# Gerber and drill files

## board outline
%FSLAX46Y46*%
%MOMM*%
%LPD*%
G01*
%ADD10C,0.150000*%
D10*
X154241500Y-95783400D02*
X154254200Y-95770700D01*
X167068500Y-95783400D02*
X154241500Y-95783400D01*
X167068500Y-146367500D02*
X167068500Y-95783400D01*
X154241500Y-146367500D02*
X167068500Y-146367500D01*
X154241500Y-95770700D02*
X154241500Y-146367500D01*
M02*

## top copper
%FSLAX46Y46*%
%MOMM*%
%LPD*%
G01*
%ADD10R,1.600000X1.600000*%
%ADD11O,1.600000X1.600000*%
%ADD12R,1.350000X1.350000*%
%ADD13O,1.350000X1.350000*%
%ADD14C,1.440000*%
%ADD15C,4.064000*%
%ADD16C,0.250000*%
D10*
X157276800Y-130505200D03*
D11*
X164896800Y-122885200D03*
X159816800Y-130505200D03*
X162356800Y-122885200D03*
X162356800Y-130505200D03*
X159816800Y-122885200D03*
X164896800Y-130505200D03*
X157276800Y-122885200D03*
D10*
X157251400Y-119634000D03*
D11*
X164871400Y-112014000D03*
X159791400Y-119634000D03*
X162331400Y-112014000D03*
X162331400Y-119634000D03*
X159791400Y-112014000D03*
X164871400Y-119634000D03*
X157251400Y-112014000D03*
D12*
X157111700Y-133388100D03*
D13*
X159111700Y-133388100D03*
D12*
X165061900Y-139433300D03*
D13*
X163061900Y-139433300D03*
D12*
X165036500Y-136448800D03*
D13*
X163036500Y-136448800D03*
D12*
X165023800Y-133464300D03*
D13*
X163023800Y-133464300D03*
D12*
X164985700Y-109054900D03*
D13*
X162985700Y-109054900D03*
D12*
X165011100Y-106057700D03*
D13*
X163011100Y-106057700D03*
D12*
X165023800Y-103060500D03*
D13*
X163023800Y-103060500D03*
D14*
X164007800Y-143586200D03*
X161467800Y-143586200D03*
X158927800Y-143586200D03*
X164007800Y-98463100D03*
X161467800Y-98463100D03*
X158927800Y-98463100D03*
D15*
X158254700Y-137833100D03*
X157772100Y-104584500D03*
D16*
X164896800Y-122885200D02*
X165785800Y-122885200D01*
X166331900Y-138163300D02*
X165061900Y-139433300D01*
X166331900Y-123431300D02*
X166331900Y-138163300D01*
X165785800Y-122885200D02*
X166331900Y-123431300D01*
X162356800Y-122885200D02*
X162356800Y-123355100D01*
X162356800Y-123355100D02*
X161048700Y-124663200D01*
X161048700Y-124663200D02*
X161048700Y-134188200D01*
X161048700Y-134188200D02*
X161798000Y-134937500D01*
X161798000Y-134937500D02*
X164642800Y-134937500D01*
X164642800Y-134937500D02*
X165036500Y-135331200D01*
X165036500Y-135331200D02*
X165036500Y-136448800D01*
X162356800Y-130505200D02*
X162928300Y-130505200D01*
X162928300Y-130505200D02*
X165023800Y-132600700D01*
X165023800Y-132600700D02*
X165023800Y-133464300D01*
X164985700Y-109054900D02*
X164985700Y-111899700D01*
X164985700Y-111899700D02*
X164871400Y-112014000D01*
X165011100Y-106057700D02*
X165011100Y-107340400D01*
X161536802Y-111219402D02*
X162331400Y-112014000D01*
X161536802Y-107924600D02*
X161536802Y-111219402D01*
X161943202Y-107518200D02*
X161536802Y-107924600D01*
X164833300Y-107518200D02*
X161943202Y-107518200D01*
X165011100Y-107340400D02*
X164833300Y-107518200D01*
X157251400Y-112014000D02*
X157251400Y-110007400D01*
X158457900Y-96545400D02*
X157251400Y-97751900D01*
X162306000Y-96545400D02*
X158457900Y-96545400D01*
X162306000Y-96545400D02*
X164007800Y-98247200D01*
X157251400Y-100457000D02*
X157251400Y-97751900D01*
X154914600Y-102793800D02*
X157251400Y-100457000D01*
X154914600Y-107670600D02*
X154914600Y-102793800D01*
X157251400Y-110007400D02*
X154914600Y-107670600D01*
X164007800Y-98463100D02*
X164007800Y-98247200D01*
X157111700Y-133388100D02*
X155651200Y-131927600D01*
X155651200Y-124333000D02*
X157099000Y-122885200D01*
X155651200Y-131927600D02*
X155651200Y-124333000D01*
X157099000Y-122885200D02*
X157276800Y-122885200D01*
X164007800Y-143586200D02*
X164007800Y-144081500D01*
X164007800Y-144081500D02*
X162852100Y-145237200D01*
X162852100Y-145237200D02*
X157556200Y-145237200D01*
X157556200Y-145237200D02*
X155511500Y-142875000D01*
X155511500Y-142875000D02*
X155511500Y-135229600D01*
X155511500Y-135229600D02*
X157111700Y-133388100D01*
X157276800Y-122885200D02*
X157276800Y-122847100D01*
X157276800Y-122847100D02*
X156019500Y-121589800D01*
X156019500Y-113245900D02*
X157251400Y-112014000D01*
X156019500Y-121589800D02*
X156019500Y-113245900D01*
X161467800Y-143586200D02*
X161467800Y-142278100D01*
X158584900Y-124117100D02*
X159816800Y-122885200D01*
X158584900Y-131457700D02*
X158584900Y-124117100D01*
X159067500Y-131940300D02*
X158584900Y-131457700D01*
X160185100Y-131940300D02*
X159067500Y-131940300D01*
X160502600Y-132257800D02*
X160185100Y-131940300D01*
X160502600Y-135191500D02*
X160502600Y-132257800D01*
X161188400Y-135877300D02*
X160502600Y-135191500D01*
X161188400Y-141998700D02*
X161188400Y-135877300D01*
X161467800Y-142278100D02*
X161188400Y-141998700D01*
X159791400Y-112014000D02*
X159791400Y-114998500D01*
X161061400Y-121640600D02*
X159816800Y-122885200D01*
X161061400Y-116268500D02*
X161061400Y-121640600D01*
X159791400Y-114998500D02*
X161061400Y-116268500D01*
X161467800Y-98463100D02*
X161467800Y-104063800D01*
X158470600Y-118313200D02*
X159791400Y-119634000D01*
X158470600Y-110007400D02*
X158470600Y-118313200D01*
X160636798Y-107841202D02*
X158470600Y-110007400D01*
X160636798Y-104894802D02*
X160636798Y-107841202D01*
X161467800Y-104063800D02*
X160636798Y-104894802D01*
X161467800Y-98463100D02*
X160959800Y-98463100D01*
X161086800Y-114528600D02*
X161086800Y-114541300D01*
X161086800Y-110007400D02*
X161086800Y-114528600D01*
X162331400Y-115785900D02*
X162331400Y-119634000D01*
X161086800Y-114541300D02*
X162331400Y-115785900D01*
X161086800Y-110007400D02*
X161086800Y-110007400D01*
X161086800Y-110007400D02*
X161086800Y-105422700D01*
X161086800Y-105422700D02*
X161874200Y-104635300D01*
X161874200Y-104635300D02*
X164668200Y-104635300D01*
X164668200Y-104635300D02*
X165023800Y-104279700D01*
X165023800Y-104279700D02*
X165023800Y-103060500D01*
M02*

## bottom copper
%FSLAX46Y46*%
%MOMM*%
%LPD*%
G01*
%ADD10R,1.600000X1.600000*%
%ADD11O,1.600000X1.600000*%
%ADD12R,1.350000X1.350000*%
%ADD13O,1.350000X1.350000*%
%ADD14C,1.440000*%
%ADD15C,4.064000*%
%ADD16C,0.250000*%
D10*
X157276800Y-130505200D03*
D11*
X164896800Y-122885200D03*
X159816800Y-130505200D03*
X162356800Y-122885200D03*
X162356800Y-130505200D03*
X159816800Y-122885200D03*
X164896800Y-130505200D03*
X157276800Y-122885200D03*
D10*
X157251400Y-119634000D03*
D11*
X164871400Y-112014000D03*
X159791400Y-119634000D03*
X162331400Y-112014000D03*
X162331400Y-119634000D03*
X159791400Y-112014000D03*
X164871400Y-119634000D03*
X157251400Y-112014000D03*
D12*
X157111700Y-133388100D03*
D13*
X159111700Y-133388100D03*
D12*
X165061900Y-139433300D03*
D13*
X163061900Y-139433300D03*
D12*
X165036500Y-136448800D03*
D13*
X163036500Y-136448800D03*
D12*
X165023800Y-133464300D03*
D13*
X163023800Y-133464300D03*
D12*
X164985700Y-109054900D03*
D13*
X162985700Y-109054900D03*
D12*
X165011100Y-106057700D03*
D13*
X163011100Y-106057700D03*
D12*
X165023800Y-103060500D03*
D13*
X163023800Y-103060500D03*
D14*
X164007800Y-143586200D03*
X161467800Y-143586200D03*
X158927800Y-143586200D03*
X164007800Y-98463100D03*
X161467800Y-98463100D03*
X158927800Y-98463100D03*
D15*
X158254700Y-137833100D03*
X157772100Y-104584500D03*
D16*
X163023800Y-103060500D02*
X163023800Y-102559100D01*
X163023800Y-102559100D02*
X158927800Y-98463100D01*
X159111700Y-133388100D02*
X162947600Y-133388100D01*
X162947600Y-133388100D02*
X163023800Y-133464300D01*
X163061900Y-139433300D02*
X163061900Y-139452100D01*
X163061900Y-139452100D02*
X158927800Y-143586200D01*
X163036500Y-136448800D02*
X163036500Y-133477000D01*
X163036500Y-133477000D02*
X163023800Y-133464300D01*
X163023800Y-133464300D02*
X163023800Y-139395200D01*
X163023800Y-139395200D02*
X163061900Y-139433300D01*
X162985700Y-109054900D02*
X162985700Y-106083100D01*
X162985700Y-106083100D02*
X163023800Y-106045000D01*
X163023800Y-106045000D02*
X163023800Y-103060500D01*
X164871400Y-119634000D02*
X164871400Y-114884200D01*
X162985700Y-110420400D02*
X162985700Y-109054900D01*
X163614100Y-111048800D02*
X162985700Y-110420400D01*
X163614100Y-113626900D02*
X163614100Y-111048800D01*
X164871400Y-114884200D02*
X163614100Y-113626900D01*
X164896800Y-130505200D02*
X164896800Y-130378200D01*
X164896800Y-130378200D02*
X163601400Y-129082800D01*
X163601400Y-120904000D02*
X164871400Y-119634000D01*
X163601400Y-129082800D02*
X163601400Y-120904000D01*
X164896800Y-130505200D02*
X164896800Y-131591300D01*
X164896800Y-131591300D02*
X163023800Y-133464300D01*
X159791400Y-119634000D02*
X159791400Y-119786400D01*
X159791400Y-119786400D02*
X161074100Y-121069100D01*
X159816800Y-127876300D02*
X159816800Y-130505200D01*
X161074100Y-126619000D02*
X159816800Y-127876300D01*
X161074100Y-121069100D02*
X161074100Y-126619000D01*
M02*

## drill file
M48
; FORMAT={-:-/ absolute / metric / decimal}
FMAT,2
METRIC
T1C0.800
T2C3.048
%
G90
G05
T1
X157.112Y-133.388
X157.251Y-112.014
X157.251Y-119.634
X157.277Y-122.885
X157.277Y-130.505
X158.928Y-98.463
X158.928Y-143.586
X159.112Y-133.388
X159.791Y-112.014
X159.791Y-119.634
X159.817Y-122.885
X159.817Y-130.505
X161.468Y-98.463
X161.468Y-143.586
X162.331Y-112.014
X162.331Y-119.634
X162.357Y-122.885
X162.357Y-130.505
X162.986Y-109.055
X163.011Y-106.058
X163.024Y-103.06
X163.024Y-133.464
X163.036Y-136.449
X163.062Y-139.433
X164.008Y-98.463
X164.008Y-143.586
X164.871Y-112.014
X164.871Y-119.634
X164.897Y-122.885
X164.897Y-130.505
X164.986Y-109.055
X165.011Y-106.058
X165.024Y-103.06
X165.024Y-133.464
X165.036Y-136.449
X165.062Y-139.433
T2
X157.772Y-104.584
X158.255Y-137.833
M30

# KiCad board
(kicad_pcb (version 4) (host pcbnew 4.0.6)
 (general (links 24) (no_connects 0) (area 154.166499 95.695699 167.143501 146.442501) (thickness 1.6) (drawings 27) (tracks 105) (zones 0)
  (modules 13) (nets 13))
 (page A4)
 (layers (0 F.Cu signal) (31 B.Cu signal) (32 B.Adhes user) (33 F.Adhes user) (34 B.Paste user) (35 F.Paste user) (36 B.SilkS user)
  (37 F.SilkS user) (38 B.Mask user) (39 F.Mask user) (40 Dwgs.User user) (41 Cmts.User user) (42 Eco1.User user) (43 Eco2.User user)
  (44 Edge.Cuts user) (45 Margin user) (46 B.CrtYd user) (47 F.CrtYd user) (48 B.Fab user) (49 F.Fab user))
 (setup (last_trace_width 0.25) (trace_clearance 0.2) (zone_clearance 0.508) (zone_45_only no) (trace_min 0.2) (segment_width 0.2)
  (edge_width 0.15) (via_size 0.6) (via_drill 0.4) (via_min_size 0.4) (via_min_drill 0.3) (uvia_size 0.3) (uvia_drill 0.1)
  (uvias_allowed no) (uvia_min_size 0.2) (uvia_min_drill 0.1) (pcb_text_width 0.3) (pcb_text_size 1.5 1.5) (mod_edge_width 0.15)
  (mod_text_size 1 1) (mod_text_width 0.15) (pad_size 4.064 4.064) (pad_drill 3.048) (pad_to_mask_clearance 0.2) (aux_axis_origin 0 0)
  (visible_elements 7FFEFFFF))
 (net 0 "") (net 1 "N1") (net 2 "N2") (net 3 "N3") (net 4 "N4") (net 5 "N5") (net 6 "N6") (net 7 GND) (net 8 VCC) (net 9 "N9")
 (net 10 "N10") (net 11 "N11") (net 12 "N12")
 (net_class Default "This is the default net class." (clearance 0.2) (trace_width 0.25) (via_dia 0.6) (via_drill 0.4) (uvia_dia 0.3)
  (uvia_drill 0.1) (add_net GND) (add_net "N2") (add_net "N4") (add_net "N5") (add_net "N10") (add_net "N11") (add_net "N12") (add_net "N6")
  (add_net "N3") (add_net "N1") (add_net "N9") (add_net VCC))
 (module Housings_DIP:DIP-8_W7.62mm (layer F.Cu) (at 157.2768 130.5052 90)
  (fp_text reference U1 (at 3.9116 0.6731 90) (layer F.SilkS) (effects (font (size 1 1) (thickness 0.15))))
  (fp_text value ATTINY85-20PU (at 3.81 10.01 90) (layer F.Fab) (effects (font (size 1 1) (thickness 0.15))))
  (pad 1 thru_hole rect (at 0 0 90) (size 1.6 1.6) (drill 0.8) (layers *.Cu *.Mask) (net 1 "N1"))
  (pad 5 thru_hole oval (at 7.62 7.62 90) (size 1.6 1.6) (drill 0.8) (layers *.Cu *.Mask) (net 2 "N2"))
  (pad 2 thru_hole oval (at 0 2.54 90) (size 1.6 1.6) (drill 0.8) (layers *.Cu *.Mask) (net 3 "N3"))
  (pad 6 thru_hole oval (at 7.62 5.08 90) (size 1.6 1.6) (drill 0.8) (layers *.Cu *.Mask) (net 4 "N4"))
  (pad 3 thru_hole oval (at 0 5.08 90) (size 1.6 1.6) (drill 0.8) (layers *.Cu *.Mask) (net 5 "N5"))
  (pad 7 thru_hole oval (at 7.62 2.54 90) (size 1.6 1.6) (drill 0.8) (layers *.Cu *.Mask) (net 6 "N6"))
  (pad 4 thru_hole oval (at 0 7.62 90) (size 1.6 1.6) (drill 0.8) (layers *.Cu *.Mask) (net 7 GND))
  (pad 8 thru_hole oval (at 7.62 0 90) (size 1.6 1.6) (drill 0.8) (layers *.Cu *.Mask) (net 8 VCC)))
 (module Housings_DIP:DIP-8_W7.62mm (layer F.Cu) (at 157.2514 119.634 90)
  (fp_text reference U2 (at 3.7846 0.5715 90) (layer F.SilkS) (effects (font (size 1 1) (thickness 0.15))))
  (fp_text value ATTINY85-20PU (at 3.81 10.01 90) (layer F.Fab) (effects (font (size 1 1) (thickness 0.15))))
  (pad 1 thru_hole rect (at 0 0 90) (size 1.6 1.6) (drill 0.8) (layers *.Cu *.Mask) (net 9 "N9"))
  (pad 5 thru_hole oval (at 7.62 7.62 90) (size 1.6 1.6) (drill 0.8) (layers *.Cu *.Mask) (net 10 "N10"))
  (pad 2 thru_hole oval (at 0 2.54 90) (size 1.6 1.6) (drill 0.8) (layers *.Cu *.Mask) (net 3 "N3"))
  (pad 6 thru_hole oval (at 7.62 5.08 90) (size 1.6 1.6) (drill 0.8) (layers *.Cu *.Mask) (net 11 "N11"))
  (pad 3 thru_hole oval (at 0 5.08 90) (size 1.6 1.6) (drill 0.8) (layers *.Cu *.Mask) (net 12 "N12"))
  (pad 7 thru_hole oval (at 7.62 2.54 90) (size 1.6 1.6) (drill 0.8) (layers *.Cu *.Mask) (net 6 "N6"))
  (pad 4 thru_hole oval (at 0 7.62 90) (size 1.6 1.6) (drill 0.8) (layers *.Cu *.Mask) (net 7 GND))
  (pad 8 thru_hole oval (at 7.62 0 90) (size 1.6 1.6) (drill 0.8) (layers *.Cu *.Mask) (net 8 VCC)))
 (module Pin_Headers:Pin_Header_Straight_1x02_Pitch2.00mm (layer F.Cu) (at 157.1117 133.3881 90)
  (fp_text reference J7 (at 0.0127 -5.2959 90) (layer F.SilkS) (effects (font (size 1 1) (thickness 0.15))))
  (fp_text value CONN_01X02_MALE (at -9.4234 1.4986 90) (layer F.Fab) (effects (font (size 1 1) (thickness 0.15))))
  (pad 1 thru_hole rect (at 0 0 90) (size 1.35 1.35) (drill 0.8) (layers *.Cu *.Mask) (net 8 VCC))
  (pad 2 thru_hole oval (at 0 2 90) (size 1.35 1.35) (drill 0.8) (layers *.Cu *.Mask) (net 7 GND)))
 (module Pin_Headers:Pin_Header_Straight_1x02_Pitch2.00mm (layer F.Cu) (at 165.0619 139.4333 270)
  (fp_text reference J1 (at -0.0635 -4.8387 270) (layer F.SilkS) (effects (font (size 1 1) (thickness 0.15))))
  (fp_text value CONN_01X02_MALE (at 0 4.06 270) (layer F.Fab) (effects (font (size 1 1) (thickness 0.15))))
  (pad 1 thru_hole rect (at 0 0 270) (size 1.35 1.35) (drill 0.8) (layers *.Cu *.Mask) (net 2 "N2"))
  (pad 2 thru_hole oval (at 0 2 270) (size 1.35 1.35) (drill 0.8) (layers *.Cu *.Mask) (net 7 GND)))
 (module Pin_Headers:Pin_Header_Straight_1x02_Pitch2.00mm (layer F.Cu) (at 165.0365 136.4488 270)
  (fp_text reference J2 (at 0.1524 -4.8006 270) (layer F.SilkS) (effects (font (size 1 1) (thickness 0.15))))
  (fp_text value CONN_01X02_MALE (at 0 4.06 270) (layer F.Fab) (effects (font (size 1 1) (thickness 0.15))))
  (pad 1 thru_hole rect (at 0 0 270) (size 1.35 1.35) (drill 0.8) (layers *.Cu *.Mask) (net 4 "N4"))
  (pad 2 thru_hole oval (at 0 2 270) (size 1.35 1.35) (drill 0.8) (layers *.Cu *.Mask) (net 7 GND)))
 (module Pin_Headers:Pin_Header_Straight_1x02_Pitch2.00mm (layer F.Cu) (at 165.0238 133.4643 270)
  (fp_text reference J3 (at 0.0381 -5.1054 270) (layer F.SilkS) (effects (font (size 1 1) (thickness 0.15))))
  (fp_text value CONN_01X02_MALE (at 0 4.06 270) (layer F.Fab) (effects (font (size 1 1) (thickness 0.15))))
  (pad 1 thru_hole rect (at 0 0 270) (size 1.35 1.35) (drill 0.8) (layers *.Cu *.Mask) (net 5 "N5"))
  (pad 2 thru_hole oval (at 0 2 270) (size 1.35 1.35) (drill 0.8) (layers *.Cu *.Mask) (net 7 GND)))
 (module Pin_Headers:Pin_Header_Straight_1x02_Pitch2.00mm (layer F.Cu) (at 164.9857 109.0549 270)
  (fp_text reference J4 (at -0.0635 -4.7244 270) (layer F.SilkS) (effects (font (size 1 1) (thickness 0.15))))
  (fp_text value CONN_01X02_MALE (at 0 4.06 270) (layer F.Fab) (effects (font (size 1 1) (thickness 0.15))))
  (pad 1 thru_hole rect (at 0 0 270) (size 1.35 1.35) (drill 0.8) (layers *.Cu *.Mask) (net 10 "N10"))
  (pad 2 thru_hole oval (at 0 2 270) (size 1.35 1.35) (drill 0.8) (layers *.Cu *.Mask) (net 7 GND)))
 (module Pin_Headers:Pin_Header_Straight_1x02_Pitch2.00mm (layer F.Cu) (at 165.0111 106.0577 270)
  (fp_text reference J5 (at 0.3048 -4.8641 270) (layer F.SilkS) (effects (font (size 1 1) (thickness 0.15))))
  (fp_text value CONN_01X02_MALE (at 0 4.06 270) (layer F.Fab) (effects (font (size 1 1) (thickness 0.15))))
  (pad 1 thru_hole rect (at 0 0 270) (size 1.35 1.35) (drill 0.8) (layers *.Cu *.Mask) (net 11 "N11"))
  (pad 2 thru_hole oval (at 0 2 270) (size 1.35 1.35) (drill 0.8) (layers *.Cu *.Mask) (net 7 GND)))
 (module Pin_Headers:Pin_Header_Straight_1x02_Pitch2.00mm (layer F.Cu) (at 165.0238 103.0605 270)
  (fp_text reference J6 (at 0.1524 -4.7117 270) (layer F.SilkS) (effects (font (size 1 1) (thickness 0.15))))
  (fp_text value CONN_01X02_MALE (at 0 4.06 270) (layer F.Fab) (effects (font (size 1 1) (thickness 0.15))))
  (pad 1 thru_hole rect (at 0 0 270) (size 1.35 1.35) (drill 0.8) (layers *.Cu *.Mask) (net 12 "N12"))
  (pad 2 thru_hole oval (at 0 2 270) (size 1.35 1.35) (drill 0.8) (layers *.Cu *.Mask) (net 7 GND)))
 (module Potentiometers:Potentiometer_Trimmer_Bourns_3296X (layer F.Cu) (at 164.0078 143.5862)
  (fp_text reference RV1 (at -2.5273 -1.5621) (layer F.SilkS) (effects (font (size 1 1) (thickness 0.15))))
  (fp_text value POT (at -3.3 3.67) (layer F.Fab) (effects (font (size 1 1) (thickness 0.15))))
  (pad 1 thru_hole circle (at 0 0) (size 1.44 1.44) (drill 0.8) (layers *.Cu *.Mask) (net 8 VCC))
  (pad 2 thru_hole circle (at -2.54 0) (size 1.44 1.44) (drill 0.8) (layers *.Cu *.Mask) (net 6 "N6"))
  (pad 3 thru_hole circle (at -5.08 0) (size 1.44 1.44) (drill 0.8) (layers *.Cu *.Mask) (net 7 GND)))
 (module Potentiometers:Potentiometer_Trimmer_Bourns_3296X (layer F.Cu) (at 164.0078 98.4631)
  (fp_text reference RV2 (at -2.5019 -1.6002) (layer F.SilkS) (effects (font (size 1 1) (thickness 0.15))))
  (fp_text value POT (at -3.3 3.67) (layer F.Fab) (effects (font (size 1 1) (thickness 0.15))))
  (pad 1 thru_hole circle (at 0 0) (size 1.44 1.44) (drill 0.8) (layers *.Cu *.Mask) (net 8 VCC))
  (pad 2 thru_hole circle (at -2.54 0) (size 1.44 1.44) (drill 0.8) (layers *.Cu *.Mask) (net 3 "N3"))
  (pad 3 thru_hole circle (at -5.08 0) (size 1.44 1.44) (drill 0.8) (layers *.Cu *.Mask) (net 7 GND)))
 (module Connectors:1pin (layer F.Cu) (at 158.2547 137.8331)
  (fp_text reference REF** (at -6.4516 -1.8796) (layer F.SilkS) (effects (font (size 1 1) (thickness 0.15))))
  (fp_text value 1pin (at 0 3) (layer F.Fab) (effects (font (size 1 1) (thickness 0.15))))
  (pad 1 thru_hole circle (at 0 0) (size 4.064 4.064) (drill 3.048) (layers *.Cu *.Mask)))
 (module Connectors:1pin (layer F.Cu) (at 157.7721 104.5845)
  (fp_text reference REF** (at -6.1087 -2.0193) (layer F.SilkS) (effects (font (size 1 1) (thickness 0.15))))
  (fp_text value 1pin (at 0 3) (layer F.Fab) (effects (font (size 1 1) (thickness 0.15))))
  (pad 1 thru_hole circle (at 0 0) (size 4.064 4.064) (drill 3.048) (layers *.Cu *.Mask)))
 (gr_line (start 154.2415 95.7834) (end 154.2542 95.7707) (angle 90) (layer Edge.Cuts) (width 0.15))
 (gr_line (start 167.0685 95.7834) (end 154.2415 95.7834) (angle 90) (layer Edge.Cuts) (width 0.15))
 (gr_line (start 167.0685 146.3675) (end 167.0685 95.7834) (angle 90) (layer Edge.Cuts) (width 0.15))
 (gr_line (start 154.2415 146.3675) (end 167.0685 146.3675) (angle 90) (layer Edge.Cuts) (width 0.15))
 (gr_line (start 154.2415 95.7707) (end 154.2415 146.3675) (angle 90) (layer Edge.Cuts) (width 0.15))
 (segment (start 164.8968 122.8852) (end 165.7858 122.8852) (width 0.25) (layer F.Cu) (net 2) (status 10))
 (segment (start 166.3319 138.1633) (end 165.0619 139.4333) (width 0.25) (layer F.Cu) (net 2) (status 20))
 (segment (start 166.3319 123.4313) (end 166.3319 138.1633) (width 0.25) (layer F.Cu) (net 2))
 (segment (start 165.7858 122.8852) (end 166.3319 123.4313) (width 0.25) (layer F.Cu) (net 2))
 (segment (start 163.0238 103.0605) (end 163.0238 102.5591) (width 0.25) (layer B.Cu) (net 7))
 (segment (start 163.0238 102.5591) (end 158.9278 98.4631) (width 0.25) (layer B.Cu) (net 7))
 (segment (start 159.1117 133.3881) (end 162.9476 133.3881) (width 0.25) (layer B.Cu) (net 7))
 (segment (start 162.9476 133.3881) (end 163.0238 133.4643) (width 0.25) (layer B.Cu) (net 7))
 (segment (start 163.0619 139.4333) (end 163.0619 139.4521) (width 0.25) (layer B.Cu) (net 7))
 (segment (start 163.0619 139.4521) (end 158.9278 143.5862) (width 0.25) (layer B.Cu) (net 7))
 (segment (start 163.0365 136.4488) (end 163.0365 133.477) (width 0.25) (layer B.Cu) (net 7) (status 30))
 (segment (start 163.0365 133.477) (end 163.0238 133.4643) (width 0.25) (layer B.Cu) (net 7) (status 30))
 (segment (start 163.0238 133.4643) (end 163.0238 139.3952) (width 0.25) (layer B.Cu) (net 7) (status 30))
 (segment (start 163.0238 139.3952) (end 163.0619 139.4333) (width 0.25) (layer B.Cu) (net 7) (status 30))
 (segment (start 162.9857 109.0549) (end 162.9857 106.0831) (width 0.25) (layer B.Cu) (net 7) (status 30))
 (segment (start 162.9857 106.0831) (end 163.0238 106.045) (width 0.25) (layer B.Cu) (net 7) (status 30))
 (segment (start 163.0238 106.045) (end 163.0238 103.0605) (width 0.25) (layer B.Cu) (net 7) (status 30))
 (segment (start 164.8714 119.634) (end 164.8714 114.8842) (width 0.25) (layer B.Cu) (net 7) (status 10))
 (segment (start 162.9857 110.4204) (end 162.9857 109.0549) (width 0.25) (layer B.Cu) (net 7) (status 20))
 (segment (start 163.6141 111.0488) (end 162.9857 110.4204) (width 0.25) (layer B.Cu) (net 7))
 (segment (start 163.6141 113.6269) (end 163.6141 111.0488) (width 0.25) (layer B.Cu) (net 7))
 (segment (start 164.8714 114.8842) (end 163.6141 113.6269) (width 0.25) (layer B.Cu) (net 7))
 (segment (start 164.8968 130.5052) (end 164.8968 130.3782) (width 0.25) (layer B.Cu) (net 7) (status 30))
 (segment (start 164.8968 130.3782) (end 163.6014 129.0828) (width 0.25) (layer B.Cu) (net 7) (status 10))
 (segment (start 163.6014 120.904) (end 164.8714 119.634) (width 0.25) (layer B.Cu) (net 7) (status 20))
 (segment (start 163.6014 129.0828) (end 163.6014 120.904) (width 0.25) (layer B.Cu) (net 7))
 (segment (start 164.8968 130.5052) (end 164.8968 131.5913) (width 0.25) (layer B.Cu) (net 7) (status 10))
 (segment (start 164.8968 131.5913) (end 163.0238 133.4643) (width 0.25) (layer B.Cu) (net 7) (status 20))
 (segment (start 162.3568 122.8852) (end 162.3568 123.3551) (width 0.25) (layer F.Cu) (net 4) (status 30))
 (segment (start 162.3568 123.3551) (end 161.0487 124.6632) (width 0.25) (layer F.Cu) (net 4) (status 10))
 (segment (start 161.0487 124.6632) (end 161.0487 134.1882) (width 0.25) (layer F.Cu) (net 4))
 (segment (start 161.0487 134.1882) (end 161.798 134.9375) (width 0.25) (layer F.Cu) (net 4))
 (segment (start 161.798 134.9375) (end 164.6428 134.9375) (width 0.25) (layer F.Cu) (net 4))
 (segment (start 164.6428 134.9375) (end 165.0365 135.3312) (width 0.25) (layer F.Cu) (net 4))
 (segment (start 165.0365 135.3312) (end 165.0365 136.4488) (width 0.25) (layer F.Cu) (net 4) (status 20))
 (segment (start 162.3568 130.5052) (end 162.9283 130.5052) (width 0.25) (layer F.Cu) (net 5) (status 30))
 (segment (start 162.9283 130.5052) (end 165.0238 132.6007) (width 0.25) (layer F.Cu) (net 5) (status 10))
 (segment (start 165.0238 132.6007) (end 165.0238 133.4643) (width 0.25) (layer F.Cu) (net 5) (status 20))
 (segment (start 164.9857 109.0549) (end 164.9857 111.8997) (width 0.25) (layer F.Cu) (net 10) (status 30))
 (segment (start 164.9857 111.8997) (end 164.8714 112.014) (width 0.25) (layer F.Cu) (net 10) (status 30))
 (segment (start 165.0111 106.0577) (end 165.0111 107.3404) (width 0.25) (layer F.Cu) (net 11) (status 10))
 (segment (start 161.536802 111.219402) (end 162.3314 112.014) (width 0.25) (layer F.Cu) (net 11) (status 20))
 (segment (start 161.536802 107.9246) (end 161.536802 111.219402) (width 0.25) (layer F.Cu) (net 11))
 (segment (start 161.943202 107.5182) (end 161.536802 107.9246) (width 0.25) (layer F.Cu) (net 11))
 (segment (start 164.8333 107.5182) (end 161.943202 107.5182) (width 0.25) (layer F.Cu) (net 11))
 (segment (start 165.0111 107.3404) (end 164.8333 107.5182) (width 0.25) (layer F.Cu) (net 11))
 (segment (start 157.2514 112.014) (end 157.2514 110.0074) (width 0.25) (layer F.Cu) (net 8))
 (segment (start 158.4579 96.5454) (end 157.2514 97.7519) (width 0.25) (layer F.Cu) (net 8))
 (segment (start 162.306 96.5454) (end 158.4579 96.5454) (width 0.25) (layer F.Cu) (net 8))
 (segment (start 162.306 96.5454) (end 164.0078 98.2472) (width 0.25) (layer F.Cu) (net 8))
 (segment (start 157.2514 100.457) (end 157.2514 97.7519) (width 0.25) (layer F.Cu) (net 8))
 (segment (start 154.9146 102.7938) (end 157.2514 100.457) (width 0.25) (layer F.Cu) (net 8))
 (segment (start 154.9146 107.6706) (end 154.9146 102.7938) (width 0.25) (layer F.Cu) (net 8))
 (segment (start 157.2514 110.0074) (end 154.9146 107.6706) (width 0.25) (layer F.Cu) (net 8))
 (segment (start 164.0078 98.4631) (end 164.0078 98.2472) (width 0.25) (layer F.Cu) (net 8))
 (segment (start 157.1117 133.3881) (end 155.6512 131.9276) (width 0.25) (layer F.Cu) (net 8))
 (segment (start 155.6512 124.333) (end 157.099 122.8852) (width 0.25) (layer F.Cu) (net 8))
 (segment (start 155.6512 131.9276) (end 155.6512 124.333) (width 0.25) (layer F.Cu) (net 8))
 (segment (start 157.099 122.8852) (end 157.2768 122.8852) (width 0.25) (layer F.Cu) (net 8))
 (segment (start 164.0078 143.5862) (end 164.0078 144.0815) (width 0.25) (layer F.Cu) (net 8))
 (segment (start 164.0078 144.0815) (end 162.8521 145.2372) (width 0.25) (layer F.Cu) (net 8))
 (segment (start 162.8521 145.2372) (end 157.5562 145.2372) (width 0.25) (layer F.Cu) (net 8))
 (segment (start 157.5562 145.2372) (end 155.5115 142.875) (width 0.25) (layer F.Cu) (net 8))
 (segment (start 155.5115 142.875) (end 155.5115 135.2296) (width 0.25) (layer F.Cu) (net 8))
 (segment (start 155.5115 135.2296) (end 157.1117 133.3881) (width 0.25) (layer F.Cu) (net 8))
 (segment (start 157.2768 122.8852) (end 157.2768 122.8471) (width 0.25) (layer F.Cu) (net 8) (status 30))
 (segment (start 157.2768 122.8471) (end 156.0195 121.5898) (width 0.25) (layer F.Cu) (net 8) (status 10))
 (segment (start 156.0195 113.2459) (end 157.2514 112.014) (width 0.25) (layer F.Cu) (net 8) (status 20))
 (segment (start 156.0195 121.5898) (end 156.0195 113.2459) (width 0.25) (layer F.Cu) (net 8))
 (segment (start 161.4678 143.5862) (end 161.4678 142.2781) (width 0.25) (layer F.Cu) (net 6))
 (segment (start 158.5849 124.1171) (end 159.8168 122.8852) (width 0.25) (layer F.Cu) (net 6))
 (segment (start 158.5849 131.4577) (end 158.5849 124.1171) (width 0.25) (layer F.Cu) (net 6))
 (segment (start 159.0675 131.9403) (end 158.5849 131.4577) (width 0.25) (layer F.Cu) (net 6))
 (segment (start 160.1851 131.9403) (end 159.0675 131.9403) (width 0.25) (layer F.Cu) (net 6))
 (segment (start 160.5026 132.2578) (end 160.1851 131.9403) (width 0.25) (layer F.Cu) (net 6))
 (segment (start 160.5026 135.1915) (end 160.5026 132.2578) (width 0.25) (layer F.Cu) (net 6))
 (segment (start 161.1884 135.8773) (end 160.5026 135.1915) (width 0.25) (layer F.Cu) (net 6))
 (segment (start 161.1884 141.9987) (end 161.1884 135.8773) (width 0.25) (layer F.Cu) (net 6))
 (segment (start 161.4678 142.2781) (end 161.1884 141.9987) (width 0.25) (layer F.Cu) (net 6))
 (segment (start 159.7914 112.014) (end 159.7914 114.9985) (width 0.25) (layer F.Cu) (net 6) (status 10))
 (segment (start 161.0614 121.6406) (end 159.8168 122.8852) (width 0.25) (layer F.Cu) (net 6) (status 20))
 (segment (start 161.0614 116.2685) (end 161.0614 121.6406) (width 0.25) (layer F.Cu) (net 6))
 (segment (start 159.7914 114.9985) (end 161.0614 116.2685) (width 0.25) (layer F.Cu) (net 6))
 (segment (start 161.4678 98.4631) (end 161.4678 104.0638) (width 0.25) (layer F.Cu) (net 3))
 (segment (start 158.4706 118.3132) (end 159.7914 119.634) (width 0.25) (layer F.Cu) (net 3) (status 20))
 (segment (start 158.4706 110.0074) (end 158.4706 118.3132) (width 0.25) (layer F.Cu) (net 3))
 (segment (start 160.636798 107.841202) (end 158.4706 110.0074) (width 0.25) (layer F.Cu) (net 3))
 (segment (start 160.636798 104.894802) (end 160.636798 107.841202) (width 0.25) (layer F.Cu) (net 3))
 (segment (start 161.4678 104.0638) (end 160.636798 104.894802) (width 0.25) (layer F.Cu) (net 3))
 (segment (start 161.4678 98.4631) (end 160.9598 98.4631) (width 0.25) (layer F.Cu) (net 3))
 (segment (start 159.7914 119.634) (end 159.7914 119.7864) (width 0.25) (layer B.Cu) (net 3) (status 30))
 (segment (start 159.7914 119.7864) (end 161.0741 121.0691) (width 0.25) (layer B.Cu) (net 3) (status 10))
 (segment (start 159.8168 127.8763) (end 159.8168 130.5052) (width 0.25) (layer B.Cu) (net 3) (status 20))
 (segment (start 161.0741 126.619) (end 159.8168 127.8763) (width 0.25) (layer B.Cu) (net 3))
 (segment (start 161.0741 121.0691) (end 161.0741 126.619) (width 0.25) (layer B.Cu) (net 3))
 (segment (start 161.0868 114.5286) (end 161.0868 114.5413) (width 0.25) (layer F.Cu) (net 12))
 (segment (start 161.0868 110.0074) (end 161.0868 114.5286) (width 0.25) (layer F.Cu) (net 12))
 (segment (start 162.3314 115.7859) (end 162.3314 119.634) (width 0.25) (layer F.Cu) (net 12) (status 20))
 (segment (start 161.0868 114.5413) (end 162.3314 115.7859) (width 0.25) (layer F.Cu) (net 12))
 (segment (start 161.0868 110.0074) (end 161.0868 110.0074) (width 0.25) (layer F.Cu) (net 12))
 (segment (start 161.0868 110.0074) (end 161.0868 105.4227) (width 0.25) (layer F.Cu) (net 12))
 (segment (start 161.0868 105.4227) (end 161.8742 104.6353) (width 0.25) (layer F.Cu) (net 12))
 (segment (start 161.8742 104.6353) (end 164.6682 104.6353) (width 0.25) (layer F.Cu) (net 12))
 (segment (start 164.6682 104.6353) (end 165.0238 104.2797) (width 0.25) (layer F.Cu) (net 12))
 (segment (start 165.0238 104.2797) (end 165.0238 103.0605) (width 0.25) (layer F.Cu) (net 12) (status 20)))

